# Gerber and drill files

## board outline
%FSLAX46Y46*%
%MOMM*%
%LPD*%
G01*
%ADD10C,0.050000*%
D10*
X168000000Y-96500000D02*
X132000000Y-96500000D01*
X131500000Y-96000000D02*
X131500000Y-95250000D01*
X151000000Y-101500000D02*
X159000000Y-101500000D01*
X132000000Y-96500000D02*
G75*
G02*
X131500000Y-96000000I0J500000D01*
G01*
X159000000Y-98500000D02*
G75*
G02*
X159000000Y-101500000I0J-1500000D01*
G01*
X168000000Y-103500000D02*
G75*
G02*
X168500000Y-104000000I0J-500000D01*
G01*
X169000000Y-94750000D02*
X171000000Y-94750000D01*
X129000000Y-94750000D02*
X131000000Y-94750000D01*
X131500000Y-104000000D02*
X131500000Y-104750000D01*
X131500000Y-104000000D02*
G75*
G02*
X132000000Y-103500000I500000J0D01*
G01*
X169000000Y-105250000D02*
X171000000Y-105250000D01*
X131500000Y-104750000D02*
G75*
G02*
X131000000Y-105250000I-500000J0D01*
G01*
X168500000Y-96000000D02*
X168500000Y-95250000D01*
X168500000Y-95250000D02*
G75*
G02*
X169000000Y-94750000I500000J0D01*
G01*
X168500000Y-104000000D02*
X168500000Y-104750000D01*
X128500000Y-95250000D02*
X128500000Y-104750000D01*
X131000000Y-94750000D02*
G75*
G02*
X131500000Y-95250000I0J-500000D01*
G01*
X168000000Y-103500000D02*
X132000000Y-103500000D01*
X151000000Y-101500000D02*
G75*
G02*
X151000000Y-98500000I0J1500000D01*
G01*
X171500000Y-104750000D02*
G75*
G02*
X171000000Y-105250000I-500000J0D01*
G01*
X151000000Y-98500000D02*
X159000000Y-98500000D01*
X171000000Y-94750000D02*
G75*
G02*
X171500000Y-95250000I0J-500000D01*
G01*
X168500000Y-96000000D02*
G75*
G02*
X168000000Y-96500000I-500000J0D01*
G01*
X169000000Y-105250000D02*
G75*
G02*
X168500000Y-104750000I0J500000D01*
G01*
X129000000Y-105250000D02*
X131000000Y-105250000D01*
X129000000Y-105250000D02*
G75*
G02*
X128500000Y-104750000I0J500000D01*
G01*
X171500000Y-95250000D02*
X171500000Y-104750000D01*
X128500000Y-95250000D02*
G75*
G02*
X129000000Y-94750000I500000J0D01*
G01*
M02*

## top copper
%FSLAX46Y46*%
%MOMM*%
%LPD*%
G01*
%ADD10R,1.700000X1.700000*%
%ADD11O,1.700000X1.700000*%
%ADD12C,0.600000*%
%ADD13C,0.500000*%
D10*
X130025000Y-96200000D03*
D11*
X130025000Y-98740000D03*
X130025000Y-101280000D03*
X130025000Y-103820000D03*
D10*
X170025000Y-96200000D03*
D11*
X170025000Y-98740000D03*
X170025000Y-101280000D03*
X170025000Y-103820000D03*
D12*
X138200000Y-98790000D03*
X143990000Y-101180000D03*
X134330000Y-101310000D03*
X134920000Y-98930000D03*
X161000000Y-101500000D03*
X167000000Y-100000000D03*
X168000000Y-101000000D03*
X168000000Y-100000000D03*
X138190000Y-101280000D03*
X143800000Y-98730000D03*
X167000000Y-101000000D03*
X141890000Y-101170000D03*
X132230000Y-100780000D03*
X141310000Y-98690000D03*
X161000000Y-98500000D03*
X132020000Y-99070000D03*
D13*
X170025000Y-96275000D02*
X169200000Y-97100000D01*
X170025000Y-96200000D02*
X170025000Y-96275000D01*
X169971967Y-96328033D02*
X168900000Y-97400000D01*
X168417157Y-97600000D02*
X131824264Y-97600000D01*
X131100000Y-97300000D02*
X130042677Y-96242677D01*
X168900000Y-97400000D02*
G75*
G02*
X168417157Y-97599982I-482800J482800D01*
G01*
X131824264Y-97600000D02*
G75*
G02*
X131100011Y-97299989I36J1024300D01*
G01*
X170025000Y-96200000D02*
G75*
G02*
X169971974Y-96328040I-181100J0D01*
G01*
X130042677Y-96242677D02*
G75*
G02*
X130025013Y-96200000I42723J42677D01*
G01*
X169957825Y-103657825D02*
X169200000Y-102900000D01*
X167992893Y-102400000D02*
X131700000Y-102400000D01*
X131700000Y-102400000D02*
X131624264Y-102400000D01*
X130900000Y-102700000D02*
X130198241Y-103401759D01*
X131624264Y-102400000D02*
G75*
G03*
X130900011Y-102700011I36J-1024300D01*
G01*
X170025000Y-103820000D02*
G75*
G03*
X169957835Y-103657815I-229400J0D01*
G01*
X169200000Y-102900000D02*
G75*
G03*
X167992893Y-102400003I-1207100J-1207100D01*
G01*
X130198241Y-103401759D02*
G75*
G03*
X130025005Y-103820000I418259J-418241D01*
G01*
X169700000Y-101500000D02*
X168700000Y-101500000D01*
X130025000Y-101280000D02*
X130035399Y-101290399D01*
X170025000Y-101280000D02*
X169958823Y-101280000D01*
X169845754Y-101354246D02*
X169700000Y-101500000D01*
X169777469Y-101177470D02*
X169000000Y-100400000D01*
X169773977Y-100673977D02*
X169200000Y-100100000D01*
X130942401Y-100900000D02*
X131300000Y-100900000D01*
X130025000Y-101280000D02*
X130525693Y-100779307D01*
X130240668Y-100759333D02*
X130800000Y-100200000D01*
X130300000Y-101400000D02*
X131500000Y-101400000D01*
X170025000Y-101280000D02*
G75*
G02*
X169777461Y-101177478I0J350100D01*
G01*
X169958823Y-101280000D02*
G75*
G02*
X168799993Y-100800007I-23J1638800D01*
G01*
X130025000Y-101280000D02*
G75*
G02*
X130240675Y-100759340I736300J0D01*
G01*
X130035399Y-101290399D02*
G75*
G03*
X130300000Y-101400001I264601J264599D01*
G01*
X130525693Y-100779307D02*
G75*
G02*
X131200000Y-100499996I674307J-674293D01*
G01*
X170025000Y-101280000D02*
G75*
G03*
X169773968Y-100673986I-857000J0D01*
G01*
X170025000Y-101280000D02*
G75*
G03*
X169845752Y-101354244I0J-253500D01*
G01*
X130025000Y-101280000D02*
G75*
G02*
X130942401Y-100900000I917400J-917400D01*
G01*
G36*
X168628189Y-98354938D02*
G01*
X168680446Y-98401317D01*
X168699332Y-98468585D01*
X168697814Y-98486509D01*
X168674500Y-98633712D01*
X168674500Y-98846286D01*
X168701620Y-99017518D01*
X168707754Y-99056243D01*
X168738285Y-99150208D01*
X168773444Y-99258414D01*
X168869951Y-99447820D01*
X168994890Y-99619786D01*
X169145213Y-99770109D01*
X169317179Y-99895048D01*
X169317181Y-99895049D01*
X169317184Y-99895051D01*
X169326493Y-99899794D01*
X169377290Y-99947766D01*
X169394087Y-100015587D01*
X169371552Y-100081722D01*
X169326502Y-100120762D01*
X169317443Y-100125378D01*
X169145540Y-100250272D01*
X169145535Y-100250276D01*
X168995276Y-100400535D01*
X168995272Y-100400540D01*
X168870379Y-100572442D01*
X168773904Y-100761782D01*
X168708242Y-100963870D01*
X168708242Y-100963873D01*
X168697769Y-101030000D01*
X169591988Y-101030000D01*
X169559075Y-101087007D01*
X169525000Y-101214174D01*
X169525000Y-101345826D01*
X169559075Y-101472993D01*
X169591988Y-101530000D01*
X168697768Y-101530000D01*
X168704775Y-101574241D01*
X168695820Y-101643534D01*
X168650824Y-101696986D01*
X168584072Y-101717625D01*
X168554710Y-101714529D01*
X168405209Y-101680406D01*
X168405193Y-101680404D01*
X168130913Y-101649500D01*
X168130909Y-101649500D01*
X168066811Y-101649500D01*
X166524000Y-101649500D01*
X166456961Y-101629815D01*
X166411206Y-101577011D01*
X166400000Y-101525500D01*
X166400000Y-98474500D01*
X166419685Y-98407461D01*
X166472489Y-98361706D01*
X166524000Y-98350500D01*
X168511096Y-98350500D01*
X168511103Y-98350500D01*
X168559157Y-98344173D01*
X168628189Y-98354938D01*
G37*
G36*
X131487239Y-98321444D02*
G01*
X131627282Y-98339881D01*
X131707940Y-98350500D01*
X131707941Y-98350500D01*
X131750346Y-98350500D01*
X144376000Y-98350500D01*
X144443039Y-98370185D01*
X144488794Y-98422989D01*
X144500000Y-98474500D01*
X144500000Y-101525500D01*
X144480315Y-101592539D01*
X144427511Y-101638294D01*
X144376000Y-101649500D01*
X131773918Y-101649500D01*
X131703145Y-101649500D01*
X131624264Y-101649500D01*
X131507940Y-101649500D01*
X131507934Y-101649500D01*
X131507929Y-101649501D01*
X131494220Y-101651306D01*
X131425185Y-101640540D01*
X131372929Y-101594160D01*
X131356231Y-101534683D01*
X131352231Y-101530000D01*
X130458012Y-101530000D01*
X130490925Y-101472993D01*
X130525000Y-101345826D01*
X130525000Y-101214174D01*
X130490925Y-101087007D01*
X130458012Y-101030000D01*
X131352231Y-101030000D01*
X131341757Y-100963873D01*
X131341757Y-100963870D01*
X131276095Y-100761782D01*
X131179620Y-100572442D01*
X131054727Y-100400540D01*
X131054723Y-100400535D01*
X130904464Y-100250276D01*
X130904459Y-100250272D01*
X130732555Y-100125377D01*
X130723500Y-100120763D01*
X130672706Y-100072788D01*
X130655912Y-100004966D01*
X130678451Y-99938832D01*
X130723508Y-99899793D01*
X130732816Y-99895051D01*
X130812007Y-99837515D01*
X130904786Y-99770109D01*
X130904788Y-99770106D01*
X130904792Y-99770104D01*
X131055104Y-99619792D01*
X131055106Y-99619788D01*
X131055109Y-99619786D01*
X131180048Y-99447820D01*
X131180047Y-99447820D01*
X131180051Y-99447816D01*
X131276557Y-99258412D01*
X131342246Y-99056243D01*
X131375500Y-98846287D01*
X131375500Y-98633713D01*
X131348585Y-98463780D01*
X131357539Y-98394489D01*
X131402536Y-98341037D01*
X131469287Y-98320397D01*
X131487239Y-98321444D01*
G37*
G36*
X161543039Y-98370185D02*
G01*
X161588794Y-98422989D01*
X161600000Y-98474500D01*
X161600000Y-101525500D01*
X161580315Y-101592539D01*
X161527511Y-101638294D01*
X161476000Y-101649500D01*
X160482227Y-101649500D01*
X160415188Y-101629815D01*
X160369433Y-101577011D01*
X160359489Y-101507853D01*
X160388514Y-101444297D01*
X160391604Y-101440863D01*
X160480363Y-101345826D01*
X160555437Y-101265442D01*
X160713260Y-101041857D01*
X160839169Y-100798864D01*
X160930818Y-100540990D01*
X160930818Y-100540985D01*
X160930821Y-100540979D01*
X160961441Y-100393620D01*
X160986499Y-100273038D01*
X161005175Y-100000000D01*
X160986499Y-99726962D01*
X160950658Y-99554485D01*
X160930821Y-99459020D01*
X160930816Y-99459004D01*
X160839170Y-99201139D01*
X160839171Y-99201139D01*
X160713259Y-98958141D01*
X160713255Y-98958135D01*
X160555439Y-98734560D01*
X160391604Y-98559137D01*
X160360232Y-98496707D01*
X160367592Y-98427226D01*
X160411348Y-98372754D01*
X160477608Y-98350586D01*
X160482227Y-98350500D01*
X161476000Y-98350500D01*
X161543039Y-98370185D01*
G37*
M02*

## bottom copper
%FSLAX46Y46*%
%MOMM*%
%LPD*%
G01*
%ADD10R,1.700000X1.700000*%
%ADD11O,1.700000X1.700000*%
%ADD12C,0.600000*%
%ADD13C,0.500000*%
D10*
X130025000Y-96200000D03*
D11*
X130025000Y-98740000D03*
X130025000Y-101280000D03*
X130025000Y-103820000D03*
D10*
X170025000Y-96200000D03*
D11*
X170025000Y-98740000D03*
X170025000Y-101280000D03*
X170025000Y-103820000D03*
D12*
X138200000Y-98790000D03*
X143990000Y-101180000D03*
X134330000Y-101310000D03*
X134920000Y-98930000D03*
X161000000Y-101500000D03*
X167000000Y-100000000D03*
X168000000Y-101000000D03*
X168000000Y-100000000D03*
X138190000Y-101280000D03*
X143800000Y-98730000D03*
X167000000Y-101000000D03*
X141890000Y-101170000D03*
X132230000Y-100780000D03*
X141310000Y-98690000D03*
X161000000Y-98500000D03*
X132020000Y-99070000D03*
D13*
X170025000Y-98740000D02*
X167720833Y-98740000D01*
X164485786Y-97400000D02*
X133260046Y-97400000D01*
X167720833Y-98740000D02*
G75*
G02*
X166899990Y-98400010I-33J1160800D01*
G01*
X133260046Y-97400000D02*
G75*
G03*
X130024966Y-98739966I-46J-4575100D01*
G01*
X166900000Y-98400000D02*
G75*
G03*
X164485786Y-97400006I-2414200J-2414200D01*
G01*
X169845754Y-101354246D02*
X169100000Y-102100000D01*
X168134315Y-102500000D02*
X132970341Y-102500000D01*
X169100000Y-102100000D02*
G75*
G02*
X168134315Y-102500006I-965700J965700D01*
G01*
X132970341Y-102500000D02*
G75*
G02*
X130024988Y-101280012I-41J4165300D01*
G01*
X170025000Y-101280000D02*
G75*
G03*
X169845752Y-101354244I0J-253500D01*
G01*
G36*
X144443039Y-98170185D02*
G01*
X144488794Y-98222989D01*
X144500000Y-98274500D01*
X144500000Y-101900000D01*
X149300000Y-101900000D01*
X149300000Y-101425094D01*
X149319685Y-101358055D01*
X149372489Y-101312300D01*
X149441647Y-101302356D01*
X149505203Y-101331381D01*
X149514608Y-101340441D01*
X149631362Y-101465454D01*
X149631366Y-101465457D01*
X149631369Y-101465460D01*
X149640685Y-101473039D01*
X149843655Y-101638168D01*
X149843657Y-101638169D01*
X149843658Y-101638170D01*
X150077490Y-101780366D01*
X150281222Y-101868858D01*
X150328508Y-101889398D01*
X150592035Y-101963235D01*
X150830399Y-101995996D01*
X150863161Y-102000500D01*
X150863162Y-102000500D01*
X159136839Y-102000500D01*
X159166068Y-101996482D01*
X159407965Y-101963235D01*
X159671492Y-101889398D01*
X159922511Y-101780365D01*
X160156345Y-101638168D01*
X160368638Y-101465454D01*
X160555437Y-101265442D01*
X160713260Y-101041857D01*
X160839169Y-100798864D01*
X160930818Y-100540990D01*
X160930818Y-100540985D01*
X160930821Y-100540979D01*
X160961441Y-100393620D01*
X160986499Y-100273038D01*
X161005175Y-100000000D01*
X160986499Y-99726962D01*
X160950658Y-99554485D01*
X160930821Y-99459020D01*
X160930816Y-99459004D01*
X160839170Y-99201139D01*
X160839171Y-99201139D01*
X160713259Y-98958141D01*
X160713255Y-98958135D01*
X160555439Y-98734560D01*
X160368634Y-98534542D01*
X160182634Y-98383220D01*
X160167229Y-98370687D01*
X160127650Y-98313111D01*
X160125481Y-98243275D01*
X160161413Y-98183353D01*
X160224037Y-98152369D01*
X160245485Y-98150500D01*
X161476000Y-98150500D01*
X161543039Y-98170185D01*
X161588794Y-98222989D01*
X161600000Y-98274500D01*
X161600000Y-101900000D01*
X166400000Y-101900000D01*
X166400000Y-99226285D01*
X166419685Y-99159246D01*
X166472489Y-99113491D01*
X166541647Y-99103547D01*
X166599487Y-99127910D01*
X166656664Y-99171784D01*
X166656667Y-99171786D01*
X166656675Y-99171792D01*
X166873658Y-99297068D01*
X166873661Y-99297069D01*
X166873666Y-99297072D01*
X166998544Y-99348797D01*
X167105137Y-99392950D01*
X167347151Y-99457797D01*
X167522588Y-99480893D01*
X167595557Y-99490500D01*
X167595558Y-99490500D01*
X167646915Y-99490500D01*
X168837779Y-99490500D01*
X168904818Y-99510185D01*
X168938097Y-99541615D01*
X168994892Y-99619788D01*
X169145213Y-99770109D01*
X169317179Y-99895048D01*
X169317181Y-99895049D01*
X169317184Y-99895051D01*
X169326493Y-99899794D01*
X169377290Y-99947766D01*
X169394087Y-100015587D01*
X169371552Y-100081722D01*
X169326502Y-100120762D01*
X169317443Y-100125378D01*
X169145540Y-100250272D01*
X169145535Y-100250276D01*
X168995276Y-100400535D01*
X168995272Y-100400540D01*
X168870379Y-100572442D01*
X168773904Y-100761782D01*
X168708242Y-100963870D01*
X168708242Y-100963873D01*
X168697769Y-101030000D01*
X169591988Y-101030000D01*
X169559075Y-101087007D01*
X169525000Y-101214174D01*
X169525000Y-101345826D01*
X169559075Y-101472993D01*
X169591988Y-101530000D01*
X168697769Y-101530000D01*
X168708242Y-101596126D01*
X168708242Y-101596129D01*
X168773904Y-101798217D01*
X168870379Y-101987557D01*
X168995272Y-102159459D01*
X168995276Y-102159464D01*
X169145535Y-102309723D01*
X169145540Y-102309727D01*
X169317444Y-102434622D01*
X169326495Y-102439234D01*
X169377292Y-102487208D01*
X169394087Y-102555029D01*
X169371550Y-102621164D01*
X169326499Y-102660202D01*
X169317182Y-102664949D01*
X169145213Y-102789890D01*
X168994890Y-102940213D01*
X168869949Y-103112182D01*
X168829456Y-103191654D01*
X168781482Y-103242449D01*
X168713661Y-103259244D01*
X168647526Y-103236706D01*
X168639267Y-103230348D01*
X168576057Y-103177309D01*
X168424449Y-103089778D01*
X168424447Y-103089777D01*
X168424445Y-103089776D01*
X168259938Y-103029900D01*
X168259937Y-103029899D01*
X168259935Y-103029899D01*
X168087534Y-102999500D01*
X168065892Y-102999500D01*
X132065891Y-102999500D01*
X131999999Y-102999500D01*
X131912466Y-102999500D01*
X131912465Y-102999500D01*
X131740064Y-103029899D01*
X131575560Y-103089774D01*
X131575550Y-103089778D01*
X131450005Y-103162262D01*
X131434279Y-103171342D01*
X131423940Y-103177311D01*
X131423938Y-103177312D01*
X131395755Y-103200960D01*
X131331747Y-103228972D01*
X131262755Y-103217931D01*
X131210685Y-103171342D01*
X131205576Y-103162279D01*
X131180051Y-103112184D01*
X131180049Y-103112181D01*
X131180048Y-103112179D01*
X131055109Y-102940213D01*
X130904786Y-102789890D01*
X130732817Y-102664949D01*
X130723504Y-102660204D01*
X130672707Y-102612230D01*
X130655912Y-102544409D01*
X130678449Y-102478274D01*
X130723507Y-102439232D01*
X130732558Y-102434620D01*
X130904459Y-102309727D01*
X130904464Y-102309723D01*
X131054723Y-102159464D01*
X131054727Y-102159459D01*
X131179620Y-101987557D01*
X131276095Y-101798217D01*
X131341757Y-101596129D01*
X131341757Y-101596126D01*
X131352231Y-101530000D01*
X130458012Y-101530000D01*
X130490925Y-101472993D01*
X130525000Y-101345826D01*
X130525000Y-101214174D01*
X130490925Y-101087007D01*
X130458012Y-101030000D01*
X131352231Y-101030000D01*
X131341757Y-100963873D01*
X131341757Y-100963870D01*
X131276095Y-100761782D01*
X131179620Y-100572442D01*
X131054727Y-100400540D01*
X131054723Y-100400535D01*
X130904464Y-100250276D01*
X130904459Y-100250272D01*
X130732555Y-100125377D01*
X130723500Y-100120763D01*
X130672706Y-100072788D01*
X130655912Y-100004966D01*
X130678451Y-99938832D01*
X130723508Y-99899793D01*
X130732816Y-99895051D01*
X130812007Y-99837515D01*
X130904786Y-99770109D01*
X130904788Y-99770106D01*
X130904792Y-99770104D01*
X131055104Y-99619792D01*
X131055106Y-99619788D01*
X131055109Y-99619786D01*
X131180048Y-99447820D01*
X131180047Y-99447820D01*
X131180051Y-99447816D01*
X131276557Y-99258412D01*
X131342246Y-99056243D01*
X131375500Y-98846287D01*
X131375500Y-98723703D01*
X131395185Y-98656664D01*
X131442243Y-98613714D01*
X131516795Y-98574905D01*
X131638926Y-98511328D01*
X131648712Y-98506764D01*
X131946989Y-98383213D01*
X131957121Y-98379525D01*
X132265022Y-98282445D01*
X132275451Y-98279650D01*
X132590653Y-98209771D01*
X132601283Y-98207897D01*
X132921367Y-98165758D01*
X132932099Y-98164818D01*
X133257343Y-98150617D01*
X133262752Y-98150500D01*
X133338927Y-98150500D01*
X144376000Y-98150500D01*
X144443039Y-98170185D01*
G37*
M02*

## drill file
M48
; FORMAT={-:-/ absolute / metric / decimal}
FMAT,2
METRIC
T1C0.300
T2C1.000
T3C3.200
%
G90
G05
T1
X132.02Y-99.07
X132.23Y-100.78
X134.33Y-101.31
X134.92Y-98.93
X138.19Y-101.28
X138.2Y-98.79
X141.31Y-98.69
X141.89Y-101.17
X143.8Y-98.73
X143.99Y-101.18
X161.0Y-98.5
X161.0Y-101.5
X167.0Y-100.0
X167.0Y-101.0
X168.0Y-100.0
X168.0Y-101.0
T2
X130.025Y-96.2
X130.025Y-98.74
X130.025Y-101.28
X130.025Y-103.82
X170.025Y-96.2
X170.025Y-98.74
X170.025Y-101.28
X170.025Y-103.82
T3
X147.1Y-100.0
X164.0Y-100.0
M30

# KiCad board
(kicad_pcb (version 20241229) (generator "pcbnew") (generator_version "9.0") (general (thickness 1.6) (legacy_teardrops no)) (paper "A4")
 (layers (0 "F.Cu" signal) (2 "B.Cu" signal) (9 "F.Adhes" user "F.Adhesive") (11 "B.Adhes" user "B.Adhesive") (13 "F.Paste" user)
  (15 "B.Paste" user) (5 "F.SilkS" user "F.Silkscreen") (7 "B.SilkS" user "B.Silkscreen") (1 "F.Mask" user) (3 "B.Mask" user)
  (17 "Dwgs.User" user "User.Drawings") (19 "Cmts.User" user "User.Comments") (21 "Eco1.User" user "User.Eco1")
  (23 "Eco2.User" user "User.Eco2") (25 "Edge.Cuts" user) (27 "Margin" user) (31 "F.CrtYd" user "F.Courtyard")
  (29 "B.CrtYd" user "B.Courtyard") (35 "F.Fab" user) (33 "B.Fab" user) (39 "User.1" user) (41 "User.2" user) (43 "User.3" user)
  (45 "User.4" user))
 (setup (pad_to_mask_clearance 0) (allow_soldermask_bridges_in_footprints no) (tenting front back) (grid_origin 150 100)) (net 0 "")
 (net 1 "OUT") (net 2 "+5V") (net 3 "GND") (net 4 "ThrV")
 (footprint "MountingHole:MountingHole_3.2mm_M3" (layer "F.Cu") (at 164 100 90)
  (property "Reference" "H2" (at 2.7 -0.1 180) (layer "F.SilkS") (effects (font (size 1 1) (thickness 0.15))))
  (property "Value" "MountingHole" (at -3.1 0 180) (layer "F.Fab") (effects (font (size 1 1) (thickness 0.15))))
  (pad "" np_thru_hole circle (at 0 0 90) (size 3.2 3.2) (drill 3.2) (layers "*.Cu" "*.Mask")))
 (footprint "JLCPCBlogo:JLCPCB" (layer "F.Cu") (at 137.93 100)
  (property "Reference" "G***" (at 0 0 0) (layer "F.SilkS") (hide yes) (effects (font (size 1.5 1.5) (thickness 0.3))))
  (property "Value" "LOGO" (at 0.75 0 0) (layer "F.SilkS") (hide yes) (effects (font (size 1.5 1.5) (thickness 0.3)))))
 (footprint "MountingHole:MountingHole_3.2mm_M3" (layer "F.Cu") (at 147 100)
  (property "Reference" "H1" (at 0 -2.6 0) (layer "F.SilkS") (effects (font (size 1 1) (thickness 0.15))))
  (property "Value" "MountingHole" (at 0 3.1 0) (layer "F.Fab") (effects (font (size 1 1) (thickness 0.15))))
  (pad "" np_thru_hole circle (at 0.1 0) (size 3.2 3.2) (drill 3.2) (layers "*.Cu" "*.Mask")))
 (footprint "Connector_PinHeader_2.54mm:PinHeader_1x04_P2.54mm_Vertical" (layer "B.Cu") (at 130.025 96.2 180)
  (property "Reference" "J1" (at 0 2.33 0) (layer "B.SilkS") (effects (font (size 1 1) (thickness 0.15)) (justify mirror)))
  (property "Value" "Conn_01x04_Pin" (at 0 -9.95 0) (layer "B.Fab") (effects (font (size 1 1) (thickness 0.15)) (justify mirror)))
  (pad "1" thru_hole rect (at 0 0 180) (size 1.7 1.7) (drill 1) (layers "*.Cu" "*.Mask") (remove_unused_layers no) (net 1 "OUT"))
  (pad "2" thru_hole oval (at 0 -2.54 180) (size 1.7 1.7) (drill 1) (layers "*.Cu" "*.Mask") (remove_unused_layers no) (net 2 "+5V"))
  (pad "3" thru_hole oval (at 0 -5.08 180) (size 1.7 1.7) (drill 1) (layers "*.Cu" "*.Mask") (remove_unused_layers no) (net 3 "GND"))
  (pad "4" thru_hole oval (at 0 -7.62 180) (size 1.7 1.7) (drill 1) (layers "*.Cu" "*.Mask") (remove_unused_layers no) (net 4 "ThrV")))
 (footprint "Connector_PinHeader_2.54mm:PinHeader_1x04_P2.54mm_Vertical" (layer "B.Cu") (at 170.025 96.2 180)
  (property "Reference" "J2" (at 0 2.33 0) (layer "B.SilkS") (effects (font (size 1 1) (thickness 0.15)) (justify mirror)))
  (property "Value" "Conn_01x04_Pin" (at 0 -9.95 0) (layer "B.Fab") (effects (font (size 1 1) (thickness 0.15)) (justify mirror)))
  (pad "1" thru_hole rect (at 0 0 180) (size 1.7 1.7) (drill 1) (layers "*.Cu" "*.Mask") (remove_unused_layers no) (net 1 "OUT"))
  (pad "2" thru_hole oval (at 0 -2.54 180) (size 1.7 1.7) (drill 1) (layers "*.Cu" "*.Mask") (remove_unused_layers no) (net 2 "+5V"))
  (pad "3" thru_hole oval (at 0 -5.08 180) (size 1.7 1.7) (drill 1) (layers "*.Cu" "*.Mask") (remove_unused_layers no) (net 3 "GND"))
  (pad "4" thru_hole oval (at 0 -7.62 180) (size 1.7 1.7) (drill 1) (layers "*.Cu" "*.Mask") (remove_unused_layers no) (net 4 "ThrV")))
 (gr_line (start 168 96.5) (end 132 96.5) (stroke (width 0.05) (type default)) (layer "Edge.Cuts"))
 (gr_line (start 131.5 96) (end 131.5 95.25) (stroke (width 0.05) (type default)) (layer "Edge.Cuts"))
 (gr_line (start 151 101.5) (end 159 101.5) (stroke (width 0.05) (type solid)) (layer "Edge.Cuts"))
 (gr_arc (start 132 96.5) (mid 131.646447 96.353553) (end 131.5 96) (stroke (width 0.05) (type default)) (layer "Edge.Cuts"))
 (gr_arc (start 159 98.5) (mid 160.5 100) (end 159 101.5) (stroke (width 0.05) (type solid)) (layer "Edge.Cuts"))
 (gr_arc (start 168 103.5) (mid 168.353553 103.646447) (end 168.5 104) (stroke (width 0.05) (type default)) (layer "Edge.Cuts"))
 (gr_line (start 169 94.75) (end 171 94.75) (stroke (width 0.05) (type default)) (layer "Edge.Cuts"))
 (gr_line (start 129 94.75) (end 131 94.75) (stroke (width 0.05) (type solid)) (layer "Edge.Cuts"))
 (gr_line (start 131.5 104) (end 131.5 104.75) (stroke (width 0.05) (type default)) (layer "Edge.Cuts"))
 (gr_arc (start 131.5 104) (mid 131.646447 103.646447) (end 132 103.5) (stroke (width 0.05) (type default)) (layer "Edge.Cuts"))
 (gr_line (start 169 105.25) (end 171 105.25) (stroke (width 0.05) (type default)) (layer "Edge.Cuts"))
 (gr_arc (start 131.5 104.75) (mid 131.353553 105.103553) (end 131 105.25) (stroke (width 0.05) (type default)) (layer "Edge.Cuts"))
 (gr_line (start 168.5 96) (end 168.5 95.25) (stroke (width 0.05) (type default)) (layer "Edge.Cuts"))
 (gr_arc (start 168.5 95.25) (mid 168.646447 94.896447) (end 169 94.75) (stroke (width 0.05) (type default)) (layer "Edge.Cuts"))
 (gr_line (start 168.5 104) (end 168.5 104.75) (stroke (width 0.05) (type default)) (layer "Edge.Cuts"))
 (gr_line (start 128.5 95.25) (end 128.5 104.75) (stroke (width 0.05) (type solid)) (layer "Edge.Cuts"))
 (gr_arc (start 131 94.75) (mid 131.353553 94.896447) (end 131.5 95.25) (stroke (width 0.05) (type default)) (layer "Edge.Cuts"))
 (gr_line (start 168 103.5) (end 132 103.5) (stroke (width 0.05) (type default)) (layer "Edge.Cuts"))
 (gr_arc (start 151 101.5) (mid 149.5 100) (end 151 98.5) (stroke (width 0.05) (type solid)) (layer "Edge.Cuts"))
 (gr_arc (start 171.5 104.75) (mid 171.353553 105.103553) (end 171 105.25) (stroke (width 0.05) (type default)) (layer "Edge.Cuts"))
 (gr_line (start 151 98.5) (end 159 98.5) (stroke (width 0.05) (type solid)) (layer "Edge.Cuts"))
 (gr_arc (start 171 94.75) (mid 171.353553 94.896447) (end 171.5 95.25) (stroke (width 0.05) (type default)) (layer "Edge.Cuts"))
 (gr_arc (start 168.5 96) (mid 168.353553 96.353553) (end 168 96.5) (stroke (width 0.05) (type default)) (layer "Edge.Cuts"))
 (gr_arc (start 169 105.25) (mid 168.646447 105.103553) (end 168.5 104.75) (stroke (width 0.05) (type default)) (layer "Edge.Cuts"))
 (gr_line (start 129 105.25) (end 131 105.25) (stroke (width 0.05) (type solid)) (layer "Edge.Cuts"))
 (gr_arc (start 129 105.25) (mid 128.646447 105.103553) (end 128.5 104.75) (stroke (width 0.05) (type default)) (layer "Edge.Cuts"))
 (gr_line (start 171.5 95.25) (end 171.5 104.75) (stroke (width 0.05) (type default)) (layer "Edge.Cuts"))
 (gr_arc (start 128.5 95.25) (mid 128.646447 94.896447) (end 129 94.75) (stroke (width 0.05) (type default)) (layer "Edge.Cuts"))
 (segment (start 170.025 98.74) (end 167.720833 98.74) (width 0.5) (layer "B.Cu") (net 2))
 (segment (start 164.485786 97.4) (end 133.260046 97.4) (width 0.5) (layer "B.Cu") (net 2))
 (arc (start 167.720833 98.74) (mid 167.276601 98.651637) (end 166.9 98.4) (width 0.5) (layer "B.Cu") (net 2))
 (arc (start 133.260046 97.4) (mid 131.509252 97.748255) (end 130.025 98.74) (width 0.5) (layer "B.Cu") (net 2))
 (arc (start 166.9 98.4) (mid 165.792349 97.659891) (end 164.485786 97.4) (width 0.5) (layer "B.Cu") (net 2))
 (segment (start 170.025 96.275) (end 169.2 97.1) (width 0.5) (layer "F.Cu") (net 1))
 (segment (start 170.025 96.2) (end 170.025 96.275) (width 0.5) (layer "F.Cu") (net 1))
 (segment (start 169.971967 96.328033) (end 168.9 97.4) (width 0.5) (layer "F.Cu") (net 1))
 (segment (start 168.417157 97.6) (end 131.824264 97.6) (width 0.5) (layer "F.Cu") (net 1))
 (segment (start 131.1 97.3) (end 130.042677 96.242677) (width 0.5) (layer "F.Cu") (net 1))
 (arc (start 168.9 97.4) (mid 168.678469 97.548022) (end 168.417157 97.6) (width 0.5) (layer "F.Cu") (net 1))
 (arc (start 131.824264 97.6) (mid 131.432295 97.522033) (end 131.1 97.3) (width 0.5) (layer "F.Cu") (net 1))
 (arc (start 170.025 96.2) (mid 170.011217 96.269291) (end 169.971967 96.328033) (width 0.5) (layer "F.Cu") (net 1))
 (arc (start 130.042677 96.242677) (mid 130.029594 96.223097) (end 130.025 96.2) (width 0.5) (layer "F.Cu") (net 1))
 (segment (start 169.957825 103.657825) (end 169.2 102.9) (width 0.5) (layer "F.Cu") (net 4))
 (segment (start 167.992893 102.4) (end 131.7 102.4) (width 0.5) (layer "F.Cu") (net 4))
 (segment (start 131.7 102.4) (end 131.624264 102.4) (width 0.5) (layer "F.Cu") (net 4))
 (segment (start 130.9 102.7) (end 130.198241 103.401759) (width 0.5) (layer "F.Cu") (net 4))
 (arc (start 131.624264 102.4) (mid 131.232296 102.477967) (end 130.9 102.7) (width 0.5) (layer "F.Cu") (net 4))
 (arc (start 170.025 103.82) (mid 170.007542 103.732232) (end 169.957825 103.657825) (width 0.5) (layer "F.Cu") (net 4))
 (arc (start 169.2 102.9) (mid 168.646175 102.529946) (end 167.992893 102.4) (width 0.5) (layer "F.Cu") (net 4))
 (arc (start 130.198241 103.401759) (mid 130.070024 103.59365) (end 130.025 103.82) (width 0.5) (layer "F.Cu") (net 4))
 (segment (start 169.7 101.5) (end 168.7 101.5) (width 0.5) (layer "F.Cu") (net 3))
 (segment (start 130.025 101.28) (end 130.035399 101.290399) (width 0.5) (layer "F.Cu") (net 3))
 (segment (start 170.025 101.28) (end 169.958823 101.28) (width 0.5) (layer "F.Cu") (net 3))
 (segment (start 169.845754 101.354246) (end 169.7 101.5) (width 0.5) (layer "F.Cu") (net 3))
 (segment (start 169.777469 101.17747) (end 169 100.4) (width 0.5) (layer "F.Cu") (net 3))
 (segment (start 169.773977 100.673977) (end 169.2 100.1) (width 0.5) (layer "F.Cu") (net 3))
 (segment (start 130.942401 100.9) (end 131.3 100.9) (width 0.5) (layer "F.Cu") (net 3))
 (segment (start 130.025 101.28) (end 130.525693 100.779307) (width 0.5) (layer "F.Cu") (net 3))
 (segment (start 130.240668 100.759333) (end 130.8 100.2) (width 0.5) (layer "F.Cu") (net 3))
 (segment (start 130.3 101.4) (end 131.5 101.4) (width 0.5) (layer "F.Cu") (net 3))
 (via (at 138.2 98.79) (size 0.6) (drill 0.3) (layers "F.Cu" "B.Cu") (free yes) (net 3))
 (via (at 143.99 101.18) (size 0.6) (drill 0.3) (layers "F.Cu" "B.Cu") (free yes) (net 3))
 (via (at 134.33 101.31) (size 0.6) (drill 0.3) (layers "F.Cu" "B.Cu") (free yes) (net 3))
 (via (at 134.92 98.93) (size 0.6) (drill 0.3) (layers "F.Cu" "B.Cu") (free yes) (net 3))
 (via (at 161 101.5) (size 0.6) (drill 0.3) (layers "F.Cu" "B.Cu") (free yes) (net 3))
 (via (at 167 100) (size 0.6) (drill 0.3) (layers "F.Cu" "B.Cu") (free yes) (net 3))
 (via (at 168 101) (size 0.6) (drill 0.3) (layers "F.Cu" "B.Cu") (free yes) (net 3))
 (via (at 168 100) (size 0.6) (drill 0.3) (layers "F.Cu" "B.Cu") (free yes) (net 3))
 (via (at 138.19 101.28) (size 0.6) (drill 0.3) (layers "F.Cu" "B.Cu") (free yes) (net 3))
 (via (at 143.8 98.73) (size 0.6) (drill 0.3) (layers "F.Cu" "B.Cu") (free yes) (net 3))
 (via (at 167 101) (size 0.6) (drill 0.3) (layers "F.Cu" "B.Cu") (free yes) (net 3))
 (via (at 141.89 101.17) (size 0.6) (drill 0.3) (layers "F.Cu" "B.Cu") (free yes) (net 3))
 (via (at 132.23 100.78) (size 0.6) (drill 0.3) (layers "F.Cu" "B.Cu") (free yes) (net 3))
 (via (at 141.31 98.69) (size 0.6) (drill 0.3) (layers "F.Cu" "B.Cu") (free yes) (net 3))
 (via (at 161 98.5) (size 0.6) (drill 0.3) (layers "F.Cu" "B.Cu") (free yes) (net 3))
 (via (at 132.02 99.07) (size 0.6) (drill 0.3) (layers "F.Cu" "B.Cu") (free yes) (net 3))
 (arc (start 170.025 101.28) (mid 169.891037 101.253353) (end 169.777469 101.17747) (width 0.5) (layer "F.Cu") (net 3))
 (arc (start 169.958823 101.28) (mid 169.331672 101.155252) (end 168.8 100.8) (width 0.5) (layer "F.Cu") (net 3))
 (arc (start 130.025 101.28) (mid 130.08105 100.998217) (end 130.240668 100.759333) (width 0.5) (layer "F.Cu") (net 3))
 (arc (start 130.035399 101.290399) (mid 130.156799 101.371515) (end 130.3 101.4) (width 0.5) (layer "F.Cu") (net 3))
 (arc (start 130.525693 100.779307) (mid 130.835068 100.57259) (end 131.2 100.5) (width 0.5) (layer "F.Cu") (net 3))
 (arc (start 170.025 101.28) (mid 169.959761 100.952023) (end 169.773977 100.673977) (width 0.5) (layer "F.Cu") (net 3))
 (arc (start 170.025 101.28) (mid 169.927993 101.299296) (end 169.845754 101.354246) (width 0.5) (layer "F.Cu") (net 3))
 (arc (start 130.025 101.28) (mid 130.445907 100.998759) (end 130.942401 100.9) (width 0.5) (layer "F.Cu") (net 3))
 (segment (start 169.845754 101.354246) (end 169.1 102.1) (width 0.5) (layer "B.Cu") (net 3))
 (segment (start 168.134315 102.5) (end 132.970341 102.5) (width 0.5) (layer "B.Cu") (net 3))
 (arc (start 169.1 102.1) (mid 168.65694 102.396044) (end 168.134315 102.5) (width 0.5) (layer "B.Cu") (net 3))
 (arc (start 132.970341 102.5) (mid 131.376334 102.182933) (end 130.025 101.28) (width 0.5) (layer "B.Cu") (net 3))
 (arc (start 170.025 101.28) (mid 169.927993 101.299296) (end 169.845754 101.354246) (width 0.5) (layer "B.Cu") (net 3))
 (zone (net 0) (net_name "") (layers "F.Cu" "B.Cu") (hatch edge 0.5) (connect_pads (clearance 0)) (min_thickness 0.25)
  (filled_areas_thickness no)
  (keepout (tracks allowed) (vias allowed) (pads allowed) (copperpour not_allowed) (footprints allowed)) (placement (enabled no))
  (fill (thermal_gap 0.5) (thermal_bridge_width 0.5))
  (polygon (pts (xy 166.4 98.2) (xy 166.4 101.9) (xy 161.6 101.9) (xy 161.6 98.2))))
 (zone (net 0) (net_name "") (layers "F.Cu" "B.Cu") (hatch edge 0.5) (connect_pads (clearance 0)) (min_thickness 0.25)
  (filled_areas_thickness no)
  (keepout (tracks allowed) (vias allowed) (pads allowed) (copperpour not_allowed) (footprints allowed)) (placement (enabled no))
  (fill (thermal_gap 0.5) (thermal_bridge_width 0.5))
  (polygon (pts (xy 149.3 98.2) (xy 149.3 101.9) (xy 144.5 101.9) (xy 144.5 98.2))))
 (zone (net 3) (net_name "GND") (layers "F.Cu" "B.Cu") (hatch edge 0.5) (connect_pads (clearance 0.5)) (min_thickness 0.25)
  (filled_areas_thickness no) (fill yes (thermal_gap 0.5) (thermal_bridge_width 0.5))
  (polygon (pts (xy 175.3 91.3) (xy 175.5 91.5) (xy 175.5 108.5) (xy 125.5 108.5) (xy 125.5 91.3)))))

